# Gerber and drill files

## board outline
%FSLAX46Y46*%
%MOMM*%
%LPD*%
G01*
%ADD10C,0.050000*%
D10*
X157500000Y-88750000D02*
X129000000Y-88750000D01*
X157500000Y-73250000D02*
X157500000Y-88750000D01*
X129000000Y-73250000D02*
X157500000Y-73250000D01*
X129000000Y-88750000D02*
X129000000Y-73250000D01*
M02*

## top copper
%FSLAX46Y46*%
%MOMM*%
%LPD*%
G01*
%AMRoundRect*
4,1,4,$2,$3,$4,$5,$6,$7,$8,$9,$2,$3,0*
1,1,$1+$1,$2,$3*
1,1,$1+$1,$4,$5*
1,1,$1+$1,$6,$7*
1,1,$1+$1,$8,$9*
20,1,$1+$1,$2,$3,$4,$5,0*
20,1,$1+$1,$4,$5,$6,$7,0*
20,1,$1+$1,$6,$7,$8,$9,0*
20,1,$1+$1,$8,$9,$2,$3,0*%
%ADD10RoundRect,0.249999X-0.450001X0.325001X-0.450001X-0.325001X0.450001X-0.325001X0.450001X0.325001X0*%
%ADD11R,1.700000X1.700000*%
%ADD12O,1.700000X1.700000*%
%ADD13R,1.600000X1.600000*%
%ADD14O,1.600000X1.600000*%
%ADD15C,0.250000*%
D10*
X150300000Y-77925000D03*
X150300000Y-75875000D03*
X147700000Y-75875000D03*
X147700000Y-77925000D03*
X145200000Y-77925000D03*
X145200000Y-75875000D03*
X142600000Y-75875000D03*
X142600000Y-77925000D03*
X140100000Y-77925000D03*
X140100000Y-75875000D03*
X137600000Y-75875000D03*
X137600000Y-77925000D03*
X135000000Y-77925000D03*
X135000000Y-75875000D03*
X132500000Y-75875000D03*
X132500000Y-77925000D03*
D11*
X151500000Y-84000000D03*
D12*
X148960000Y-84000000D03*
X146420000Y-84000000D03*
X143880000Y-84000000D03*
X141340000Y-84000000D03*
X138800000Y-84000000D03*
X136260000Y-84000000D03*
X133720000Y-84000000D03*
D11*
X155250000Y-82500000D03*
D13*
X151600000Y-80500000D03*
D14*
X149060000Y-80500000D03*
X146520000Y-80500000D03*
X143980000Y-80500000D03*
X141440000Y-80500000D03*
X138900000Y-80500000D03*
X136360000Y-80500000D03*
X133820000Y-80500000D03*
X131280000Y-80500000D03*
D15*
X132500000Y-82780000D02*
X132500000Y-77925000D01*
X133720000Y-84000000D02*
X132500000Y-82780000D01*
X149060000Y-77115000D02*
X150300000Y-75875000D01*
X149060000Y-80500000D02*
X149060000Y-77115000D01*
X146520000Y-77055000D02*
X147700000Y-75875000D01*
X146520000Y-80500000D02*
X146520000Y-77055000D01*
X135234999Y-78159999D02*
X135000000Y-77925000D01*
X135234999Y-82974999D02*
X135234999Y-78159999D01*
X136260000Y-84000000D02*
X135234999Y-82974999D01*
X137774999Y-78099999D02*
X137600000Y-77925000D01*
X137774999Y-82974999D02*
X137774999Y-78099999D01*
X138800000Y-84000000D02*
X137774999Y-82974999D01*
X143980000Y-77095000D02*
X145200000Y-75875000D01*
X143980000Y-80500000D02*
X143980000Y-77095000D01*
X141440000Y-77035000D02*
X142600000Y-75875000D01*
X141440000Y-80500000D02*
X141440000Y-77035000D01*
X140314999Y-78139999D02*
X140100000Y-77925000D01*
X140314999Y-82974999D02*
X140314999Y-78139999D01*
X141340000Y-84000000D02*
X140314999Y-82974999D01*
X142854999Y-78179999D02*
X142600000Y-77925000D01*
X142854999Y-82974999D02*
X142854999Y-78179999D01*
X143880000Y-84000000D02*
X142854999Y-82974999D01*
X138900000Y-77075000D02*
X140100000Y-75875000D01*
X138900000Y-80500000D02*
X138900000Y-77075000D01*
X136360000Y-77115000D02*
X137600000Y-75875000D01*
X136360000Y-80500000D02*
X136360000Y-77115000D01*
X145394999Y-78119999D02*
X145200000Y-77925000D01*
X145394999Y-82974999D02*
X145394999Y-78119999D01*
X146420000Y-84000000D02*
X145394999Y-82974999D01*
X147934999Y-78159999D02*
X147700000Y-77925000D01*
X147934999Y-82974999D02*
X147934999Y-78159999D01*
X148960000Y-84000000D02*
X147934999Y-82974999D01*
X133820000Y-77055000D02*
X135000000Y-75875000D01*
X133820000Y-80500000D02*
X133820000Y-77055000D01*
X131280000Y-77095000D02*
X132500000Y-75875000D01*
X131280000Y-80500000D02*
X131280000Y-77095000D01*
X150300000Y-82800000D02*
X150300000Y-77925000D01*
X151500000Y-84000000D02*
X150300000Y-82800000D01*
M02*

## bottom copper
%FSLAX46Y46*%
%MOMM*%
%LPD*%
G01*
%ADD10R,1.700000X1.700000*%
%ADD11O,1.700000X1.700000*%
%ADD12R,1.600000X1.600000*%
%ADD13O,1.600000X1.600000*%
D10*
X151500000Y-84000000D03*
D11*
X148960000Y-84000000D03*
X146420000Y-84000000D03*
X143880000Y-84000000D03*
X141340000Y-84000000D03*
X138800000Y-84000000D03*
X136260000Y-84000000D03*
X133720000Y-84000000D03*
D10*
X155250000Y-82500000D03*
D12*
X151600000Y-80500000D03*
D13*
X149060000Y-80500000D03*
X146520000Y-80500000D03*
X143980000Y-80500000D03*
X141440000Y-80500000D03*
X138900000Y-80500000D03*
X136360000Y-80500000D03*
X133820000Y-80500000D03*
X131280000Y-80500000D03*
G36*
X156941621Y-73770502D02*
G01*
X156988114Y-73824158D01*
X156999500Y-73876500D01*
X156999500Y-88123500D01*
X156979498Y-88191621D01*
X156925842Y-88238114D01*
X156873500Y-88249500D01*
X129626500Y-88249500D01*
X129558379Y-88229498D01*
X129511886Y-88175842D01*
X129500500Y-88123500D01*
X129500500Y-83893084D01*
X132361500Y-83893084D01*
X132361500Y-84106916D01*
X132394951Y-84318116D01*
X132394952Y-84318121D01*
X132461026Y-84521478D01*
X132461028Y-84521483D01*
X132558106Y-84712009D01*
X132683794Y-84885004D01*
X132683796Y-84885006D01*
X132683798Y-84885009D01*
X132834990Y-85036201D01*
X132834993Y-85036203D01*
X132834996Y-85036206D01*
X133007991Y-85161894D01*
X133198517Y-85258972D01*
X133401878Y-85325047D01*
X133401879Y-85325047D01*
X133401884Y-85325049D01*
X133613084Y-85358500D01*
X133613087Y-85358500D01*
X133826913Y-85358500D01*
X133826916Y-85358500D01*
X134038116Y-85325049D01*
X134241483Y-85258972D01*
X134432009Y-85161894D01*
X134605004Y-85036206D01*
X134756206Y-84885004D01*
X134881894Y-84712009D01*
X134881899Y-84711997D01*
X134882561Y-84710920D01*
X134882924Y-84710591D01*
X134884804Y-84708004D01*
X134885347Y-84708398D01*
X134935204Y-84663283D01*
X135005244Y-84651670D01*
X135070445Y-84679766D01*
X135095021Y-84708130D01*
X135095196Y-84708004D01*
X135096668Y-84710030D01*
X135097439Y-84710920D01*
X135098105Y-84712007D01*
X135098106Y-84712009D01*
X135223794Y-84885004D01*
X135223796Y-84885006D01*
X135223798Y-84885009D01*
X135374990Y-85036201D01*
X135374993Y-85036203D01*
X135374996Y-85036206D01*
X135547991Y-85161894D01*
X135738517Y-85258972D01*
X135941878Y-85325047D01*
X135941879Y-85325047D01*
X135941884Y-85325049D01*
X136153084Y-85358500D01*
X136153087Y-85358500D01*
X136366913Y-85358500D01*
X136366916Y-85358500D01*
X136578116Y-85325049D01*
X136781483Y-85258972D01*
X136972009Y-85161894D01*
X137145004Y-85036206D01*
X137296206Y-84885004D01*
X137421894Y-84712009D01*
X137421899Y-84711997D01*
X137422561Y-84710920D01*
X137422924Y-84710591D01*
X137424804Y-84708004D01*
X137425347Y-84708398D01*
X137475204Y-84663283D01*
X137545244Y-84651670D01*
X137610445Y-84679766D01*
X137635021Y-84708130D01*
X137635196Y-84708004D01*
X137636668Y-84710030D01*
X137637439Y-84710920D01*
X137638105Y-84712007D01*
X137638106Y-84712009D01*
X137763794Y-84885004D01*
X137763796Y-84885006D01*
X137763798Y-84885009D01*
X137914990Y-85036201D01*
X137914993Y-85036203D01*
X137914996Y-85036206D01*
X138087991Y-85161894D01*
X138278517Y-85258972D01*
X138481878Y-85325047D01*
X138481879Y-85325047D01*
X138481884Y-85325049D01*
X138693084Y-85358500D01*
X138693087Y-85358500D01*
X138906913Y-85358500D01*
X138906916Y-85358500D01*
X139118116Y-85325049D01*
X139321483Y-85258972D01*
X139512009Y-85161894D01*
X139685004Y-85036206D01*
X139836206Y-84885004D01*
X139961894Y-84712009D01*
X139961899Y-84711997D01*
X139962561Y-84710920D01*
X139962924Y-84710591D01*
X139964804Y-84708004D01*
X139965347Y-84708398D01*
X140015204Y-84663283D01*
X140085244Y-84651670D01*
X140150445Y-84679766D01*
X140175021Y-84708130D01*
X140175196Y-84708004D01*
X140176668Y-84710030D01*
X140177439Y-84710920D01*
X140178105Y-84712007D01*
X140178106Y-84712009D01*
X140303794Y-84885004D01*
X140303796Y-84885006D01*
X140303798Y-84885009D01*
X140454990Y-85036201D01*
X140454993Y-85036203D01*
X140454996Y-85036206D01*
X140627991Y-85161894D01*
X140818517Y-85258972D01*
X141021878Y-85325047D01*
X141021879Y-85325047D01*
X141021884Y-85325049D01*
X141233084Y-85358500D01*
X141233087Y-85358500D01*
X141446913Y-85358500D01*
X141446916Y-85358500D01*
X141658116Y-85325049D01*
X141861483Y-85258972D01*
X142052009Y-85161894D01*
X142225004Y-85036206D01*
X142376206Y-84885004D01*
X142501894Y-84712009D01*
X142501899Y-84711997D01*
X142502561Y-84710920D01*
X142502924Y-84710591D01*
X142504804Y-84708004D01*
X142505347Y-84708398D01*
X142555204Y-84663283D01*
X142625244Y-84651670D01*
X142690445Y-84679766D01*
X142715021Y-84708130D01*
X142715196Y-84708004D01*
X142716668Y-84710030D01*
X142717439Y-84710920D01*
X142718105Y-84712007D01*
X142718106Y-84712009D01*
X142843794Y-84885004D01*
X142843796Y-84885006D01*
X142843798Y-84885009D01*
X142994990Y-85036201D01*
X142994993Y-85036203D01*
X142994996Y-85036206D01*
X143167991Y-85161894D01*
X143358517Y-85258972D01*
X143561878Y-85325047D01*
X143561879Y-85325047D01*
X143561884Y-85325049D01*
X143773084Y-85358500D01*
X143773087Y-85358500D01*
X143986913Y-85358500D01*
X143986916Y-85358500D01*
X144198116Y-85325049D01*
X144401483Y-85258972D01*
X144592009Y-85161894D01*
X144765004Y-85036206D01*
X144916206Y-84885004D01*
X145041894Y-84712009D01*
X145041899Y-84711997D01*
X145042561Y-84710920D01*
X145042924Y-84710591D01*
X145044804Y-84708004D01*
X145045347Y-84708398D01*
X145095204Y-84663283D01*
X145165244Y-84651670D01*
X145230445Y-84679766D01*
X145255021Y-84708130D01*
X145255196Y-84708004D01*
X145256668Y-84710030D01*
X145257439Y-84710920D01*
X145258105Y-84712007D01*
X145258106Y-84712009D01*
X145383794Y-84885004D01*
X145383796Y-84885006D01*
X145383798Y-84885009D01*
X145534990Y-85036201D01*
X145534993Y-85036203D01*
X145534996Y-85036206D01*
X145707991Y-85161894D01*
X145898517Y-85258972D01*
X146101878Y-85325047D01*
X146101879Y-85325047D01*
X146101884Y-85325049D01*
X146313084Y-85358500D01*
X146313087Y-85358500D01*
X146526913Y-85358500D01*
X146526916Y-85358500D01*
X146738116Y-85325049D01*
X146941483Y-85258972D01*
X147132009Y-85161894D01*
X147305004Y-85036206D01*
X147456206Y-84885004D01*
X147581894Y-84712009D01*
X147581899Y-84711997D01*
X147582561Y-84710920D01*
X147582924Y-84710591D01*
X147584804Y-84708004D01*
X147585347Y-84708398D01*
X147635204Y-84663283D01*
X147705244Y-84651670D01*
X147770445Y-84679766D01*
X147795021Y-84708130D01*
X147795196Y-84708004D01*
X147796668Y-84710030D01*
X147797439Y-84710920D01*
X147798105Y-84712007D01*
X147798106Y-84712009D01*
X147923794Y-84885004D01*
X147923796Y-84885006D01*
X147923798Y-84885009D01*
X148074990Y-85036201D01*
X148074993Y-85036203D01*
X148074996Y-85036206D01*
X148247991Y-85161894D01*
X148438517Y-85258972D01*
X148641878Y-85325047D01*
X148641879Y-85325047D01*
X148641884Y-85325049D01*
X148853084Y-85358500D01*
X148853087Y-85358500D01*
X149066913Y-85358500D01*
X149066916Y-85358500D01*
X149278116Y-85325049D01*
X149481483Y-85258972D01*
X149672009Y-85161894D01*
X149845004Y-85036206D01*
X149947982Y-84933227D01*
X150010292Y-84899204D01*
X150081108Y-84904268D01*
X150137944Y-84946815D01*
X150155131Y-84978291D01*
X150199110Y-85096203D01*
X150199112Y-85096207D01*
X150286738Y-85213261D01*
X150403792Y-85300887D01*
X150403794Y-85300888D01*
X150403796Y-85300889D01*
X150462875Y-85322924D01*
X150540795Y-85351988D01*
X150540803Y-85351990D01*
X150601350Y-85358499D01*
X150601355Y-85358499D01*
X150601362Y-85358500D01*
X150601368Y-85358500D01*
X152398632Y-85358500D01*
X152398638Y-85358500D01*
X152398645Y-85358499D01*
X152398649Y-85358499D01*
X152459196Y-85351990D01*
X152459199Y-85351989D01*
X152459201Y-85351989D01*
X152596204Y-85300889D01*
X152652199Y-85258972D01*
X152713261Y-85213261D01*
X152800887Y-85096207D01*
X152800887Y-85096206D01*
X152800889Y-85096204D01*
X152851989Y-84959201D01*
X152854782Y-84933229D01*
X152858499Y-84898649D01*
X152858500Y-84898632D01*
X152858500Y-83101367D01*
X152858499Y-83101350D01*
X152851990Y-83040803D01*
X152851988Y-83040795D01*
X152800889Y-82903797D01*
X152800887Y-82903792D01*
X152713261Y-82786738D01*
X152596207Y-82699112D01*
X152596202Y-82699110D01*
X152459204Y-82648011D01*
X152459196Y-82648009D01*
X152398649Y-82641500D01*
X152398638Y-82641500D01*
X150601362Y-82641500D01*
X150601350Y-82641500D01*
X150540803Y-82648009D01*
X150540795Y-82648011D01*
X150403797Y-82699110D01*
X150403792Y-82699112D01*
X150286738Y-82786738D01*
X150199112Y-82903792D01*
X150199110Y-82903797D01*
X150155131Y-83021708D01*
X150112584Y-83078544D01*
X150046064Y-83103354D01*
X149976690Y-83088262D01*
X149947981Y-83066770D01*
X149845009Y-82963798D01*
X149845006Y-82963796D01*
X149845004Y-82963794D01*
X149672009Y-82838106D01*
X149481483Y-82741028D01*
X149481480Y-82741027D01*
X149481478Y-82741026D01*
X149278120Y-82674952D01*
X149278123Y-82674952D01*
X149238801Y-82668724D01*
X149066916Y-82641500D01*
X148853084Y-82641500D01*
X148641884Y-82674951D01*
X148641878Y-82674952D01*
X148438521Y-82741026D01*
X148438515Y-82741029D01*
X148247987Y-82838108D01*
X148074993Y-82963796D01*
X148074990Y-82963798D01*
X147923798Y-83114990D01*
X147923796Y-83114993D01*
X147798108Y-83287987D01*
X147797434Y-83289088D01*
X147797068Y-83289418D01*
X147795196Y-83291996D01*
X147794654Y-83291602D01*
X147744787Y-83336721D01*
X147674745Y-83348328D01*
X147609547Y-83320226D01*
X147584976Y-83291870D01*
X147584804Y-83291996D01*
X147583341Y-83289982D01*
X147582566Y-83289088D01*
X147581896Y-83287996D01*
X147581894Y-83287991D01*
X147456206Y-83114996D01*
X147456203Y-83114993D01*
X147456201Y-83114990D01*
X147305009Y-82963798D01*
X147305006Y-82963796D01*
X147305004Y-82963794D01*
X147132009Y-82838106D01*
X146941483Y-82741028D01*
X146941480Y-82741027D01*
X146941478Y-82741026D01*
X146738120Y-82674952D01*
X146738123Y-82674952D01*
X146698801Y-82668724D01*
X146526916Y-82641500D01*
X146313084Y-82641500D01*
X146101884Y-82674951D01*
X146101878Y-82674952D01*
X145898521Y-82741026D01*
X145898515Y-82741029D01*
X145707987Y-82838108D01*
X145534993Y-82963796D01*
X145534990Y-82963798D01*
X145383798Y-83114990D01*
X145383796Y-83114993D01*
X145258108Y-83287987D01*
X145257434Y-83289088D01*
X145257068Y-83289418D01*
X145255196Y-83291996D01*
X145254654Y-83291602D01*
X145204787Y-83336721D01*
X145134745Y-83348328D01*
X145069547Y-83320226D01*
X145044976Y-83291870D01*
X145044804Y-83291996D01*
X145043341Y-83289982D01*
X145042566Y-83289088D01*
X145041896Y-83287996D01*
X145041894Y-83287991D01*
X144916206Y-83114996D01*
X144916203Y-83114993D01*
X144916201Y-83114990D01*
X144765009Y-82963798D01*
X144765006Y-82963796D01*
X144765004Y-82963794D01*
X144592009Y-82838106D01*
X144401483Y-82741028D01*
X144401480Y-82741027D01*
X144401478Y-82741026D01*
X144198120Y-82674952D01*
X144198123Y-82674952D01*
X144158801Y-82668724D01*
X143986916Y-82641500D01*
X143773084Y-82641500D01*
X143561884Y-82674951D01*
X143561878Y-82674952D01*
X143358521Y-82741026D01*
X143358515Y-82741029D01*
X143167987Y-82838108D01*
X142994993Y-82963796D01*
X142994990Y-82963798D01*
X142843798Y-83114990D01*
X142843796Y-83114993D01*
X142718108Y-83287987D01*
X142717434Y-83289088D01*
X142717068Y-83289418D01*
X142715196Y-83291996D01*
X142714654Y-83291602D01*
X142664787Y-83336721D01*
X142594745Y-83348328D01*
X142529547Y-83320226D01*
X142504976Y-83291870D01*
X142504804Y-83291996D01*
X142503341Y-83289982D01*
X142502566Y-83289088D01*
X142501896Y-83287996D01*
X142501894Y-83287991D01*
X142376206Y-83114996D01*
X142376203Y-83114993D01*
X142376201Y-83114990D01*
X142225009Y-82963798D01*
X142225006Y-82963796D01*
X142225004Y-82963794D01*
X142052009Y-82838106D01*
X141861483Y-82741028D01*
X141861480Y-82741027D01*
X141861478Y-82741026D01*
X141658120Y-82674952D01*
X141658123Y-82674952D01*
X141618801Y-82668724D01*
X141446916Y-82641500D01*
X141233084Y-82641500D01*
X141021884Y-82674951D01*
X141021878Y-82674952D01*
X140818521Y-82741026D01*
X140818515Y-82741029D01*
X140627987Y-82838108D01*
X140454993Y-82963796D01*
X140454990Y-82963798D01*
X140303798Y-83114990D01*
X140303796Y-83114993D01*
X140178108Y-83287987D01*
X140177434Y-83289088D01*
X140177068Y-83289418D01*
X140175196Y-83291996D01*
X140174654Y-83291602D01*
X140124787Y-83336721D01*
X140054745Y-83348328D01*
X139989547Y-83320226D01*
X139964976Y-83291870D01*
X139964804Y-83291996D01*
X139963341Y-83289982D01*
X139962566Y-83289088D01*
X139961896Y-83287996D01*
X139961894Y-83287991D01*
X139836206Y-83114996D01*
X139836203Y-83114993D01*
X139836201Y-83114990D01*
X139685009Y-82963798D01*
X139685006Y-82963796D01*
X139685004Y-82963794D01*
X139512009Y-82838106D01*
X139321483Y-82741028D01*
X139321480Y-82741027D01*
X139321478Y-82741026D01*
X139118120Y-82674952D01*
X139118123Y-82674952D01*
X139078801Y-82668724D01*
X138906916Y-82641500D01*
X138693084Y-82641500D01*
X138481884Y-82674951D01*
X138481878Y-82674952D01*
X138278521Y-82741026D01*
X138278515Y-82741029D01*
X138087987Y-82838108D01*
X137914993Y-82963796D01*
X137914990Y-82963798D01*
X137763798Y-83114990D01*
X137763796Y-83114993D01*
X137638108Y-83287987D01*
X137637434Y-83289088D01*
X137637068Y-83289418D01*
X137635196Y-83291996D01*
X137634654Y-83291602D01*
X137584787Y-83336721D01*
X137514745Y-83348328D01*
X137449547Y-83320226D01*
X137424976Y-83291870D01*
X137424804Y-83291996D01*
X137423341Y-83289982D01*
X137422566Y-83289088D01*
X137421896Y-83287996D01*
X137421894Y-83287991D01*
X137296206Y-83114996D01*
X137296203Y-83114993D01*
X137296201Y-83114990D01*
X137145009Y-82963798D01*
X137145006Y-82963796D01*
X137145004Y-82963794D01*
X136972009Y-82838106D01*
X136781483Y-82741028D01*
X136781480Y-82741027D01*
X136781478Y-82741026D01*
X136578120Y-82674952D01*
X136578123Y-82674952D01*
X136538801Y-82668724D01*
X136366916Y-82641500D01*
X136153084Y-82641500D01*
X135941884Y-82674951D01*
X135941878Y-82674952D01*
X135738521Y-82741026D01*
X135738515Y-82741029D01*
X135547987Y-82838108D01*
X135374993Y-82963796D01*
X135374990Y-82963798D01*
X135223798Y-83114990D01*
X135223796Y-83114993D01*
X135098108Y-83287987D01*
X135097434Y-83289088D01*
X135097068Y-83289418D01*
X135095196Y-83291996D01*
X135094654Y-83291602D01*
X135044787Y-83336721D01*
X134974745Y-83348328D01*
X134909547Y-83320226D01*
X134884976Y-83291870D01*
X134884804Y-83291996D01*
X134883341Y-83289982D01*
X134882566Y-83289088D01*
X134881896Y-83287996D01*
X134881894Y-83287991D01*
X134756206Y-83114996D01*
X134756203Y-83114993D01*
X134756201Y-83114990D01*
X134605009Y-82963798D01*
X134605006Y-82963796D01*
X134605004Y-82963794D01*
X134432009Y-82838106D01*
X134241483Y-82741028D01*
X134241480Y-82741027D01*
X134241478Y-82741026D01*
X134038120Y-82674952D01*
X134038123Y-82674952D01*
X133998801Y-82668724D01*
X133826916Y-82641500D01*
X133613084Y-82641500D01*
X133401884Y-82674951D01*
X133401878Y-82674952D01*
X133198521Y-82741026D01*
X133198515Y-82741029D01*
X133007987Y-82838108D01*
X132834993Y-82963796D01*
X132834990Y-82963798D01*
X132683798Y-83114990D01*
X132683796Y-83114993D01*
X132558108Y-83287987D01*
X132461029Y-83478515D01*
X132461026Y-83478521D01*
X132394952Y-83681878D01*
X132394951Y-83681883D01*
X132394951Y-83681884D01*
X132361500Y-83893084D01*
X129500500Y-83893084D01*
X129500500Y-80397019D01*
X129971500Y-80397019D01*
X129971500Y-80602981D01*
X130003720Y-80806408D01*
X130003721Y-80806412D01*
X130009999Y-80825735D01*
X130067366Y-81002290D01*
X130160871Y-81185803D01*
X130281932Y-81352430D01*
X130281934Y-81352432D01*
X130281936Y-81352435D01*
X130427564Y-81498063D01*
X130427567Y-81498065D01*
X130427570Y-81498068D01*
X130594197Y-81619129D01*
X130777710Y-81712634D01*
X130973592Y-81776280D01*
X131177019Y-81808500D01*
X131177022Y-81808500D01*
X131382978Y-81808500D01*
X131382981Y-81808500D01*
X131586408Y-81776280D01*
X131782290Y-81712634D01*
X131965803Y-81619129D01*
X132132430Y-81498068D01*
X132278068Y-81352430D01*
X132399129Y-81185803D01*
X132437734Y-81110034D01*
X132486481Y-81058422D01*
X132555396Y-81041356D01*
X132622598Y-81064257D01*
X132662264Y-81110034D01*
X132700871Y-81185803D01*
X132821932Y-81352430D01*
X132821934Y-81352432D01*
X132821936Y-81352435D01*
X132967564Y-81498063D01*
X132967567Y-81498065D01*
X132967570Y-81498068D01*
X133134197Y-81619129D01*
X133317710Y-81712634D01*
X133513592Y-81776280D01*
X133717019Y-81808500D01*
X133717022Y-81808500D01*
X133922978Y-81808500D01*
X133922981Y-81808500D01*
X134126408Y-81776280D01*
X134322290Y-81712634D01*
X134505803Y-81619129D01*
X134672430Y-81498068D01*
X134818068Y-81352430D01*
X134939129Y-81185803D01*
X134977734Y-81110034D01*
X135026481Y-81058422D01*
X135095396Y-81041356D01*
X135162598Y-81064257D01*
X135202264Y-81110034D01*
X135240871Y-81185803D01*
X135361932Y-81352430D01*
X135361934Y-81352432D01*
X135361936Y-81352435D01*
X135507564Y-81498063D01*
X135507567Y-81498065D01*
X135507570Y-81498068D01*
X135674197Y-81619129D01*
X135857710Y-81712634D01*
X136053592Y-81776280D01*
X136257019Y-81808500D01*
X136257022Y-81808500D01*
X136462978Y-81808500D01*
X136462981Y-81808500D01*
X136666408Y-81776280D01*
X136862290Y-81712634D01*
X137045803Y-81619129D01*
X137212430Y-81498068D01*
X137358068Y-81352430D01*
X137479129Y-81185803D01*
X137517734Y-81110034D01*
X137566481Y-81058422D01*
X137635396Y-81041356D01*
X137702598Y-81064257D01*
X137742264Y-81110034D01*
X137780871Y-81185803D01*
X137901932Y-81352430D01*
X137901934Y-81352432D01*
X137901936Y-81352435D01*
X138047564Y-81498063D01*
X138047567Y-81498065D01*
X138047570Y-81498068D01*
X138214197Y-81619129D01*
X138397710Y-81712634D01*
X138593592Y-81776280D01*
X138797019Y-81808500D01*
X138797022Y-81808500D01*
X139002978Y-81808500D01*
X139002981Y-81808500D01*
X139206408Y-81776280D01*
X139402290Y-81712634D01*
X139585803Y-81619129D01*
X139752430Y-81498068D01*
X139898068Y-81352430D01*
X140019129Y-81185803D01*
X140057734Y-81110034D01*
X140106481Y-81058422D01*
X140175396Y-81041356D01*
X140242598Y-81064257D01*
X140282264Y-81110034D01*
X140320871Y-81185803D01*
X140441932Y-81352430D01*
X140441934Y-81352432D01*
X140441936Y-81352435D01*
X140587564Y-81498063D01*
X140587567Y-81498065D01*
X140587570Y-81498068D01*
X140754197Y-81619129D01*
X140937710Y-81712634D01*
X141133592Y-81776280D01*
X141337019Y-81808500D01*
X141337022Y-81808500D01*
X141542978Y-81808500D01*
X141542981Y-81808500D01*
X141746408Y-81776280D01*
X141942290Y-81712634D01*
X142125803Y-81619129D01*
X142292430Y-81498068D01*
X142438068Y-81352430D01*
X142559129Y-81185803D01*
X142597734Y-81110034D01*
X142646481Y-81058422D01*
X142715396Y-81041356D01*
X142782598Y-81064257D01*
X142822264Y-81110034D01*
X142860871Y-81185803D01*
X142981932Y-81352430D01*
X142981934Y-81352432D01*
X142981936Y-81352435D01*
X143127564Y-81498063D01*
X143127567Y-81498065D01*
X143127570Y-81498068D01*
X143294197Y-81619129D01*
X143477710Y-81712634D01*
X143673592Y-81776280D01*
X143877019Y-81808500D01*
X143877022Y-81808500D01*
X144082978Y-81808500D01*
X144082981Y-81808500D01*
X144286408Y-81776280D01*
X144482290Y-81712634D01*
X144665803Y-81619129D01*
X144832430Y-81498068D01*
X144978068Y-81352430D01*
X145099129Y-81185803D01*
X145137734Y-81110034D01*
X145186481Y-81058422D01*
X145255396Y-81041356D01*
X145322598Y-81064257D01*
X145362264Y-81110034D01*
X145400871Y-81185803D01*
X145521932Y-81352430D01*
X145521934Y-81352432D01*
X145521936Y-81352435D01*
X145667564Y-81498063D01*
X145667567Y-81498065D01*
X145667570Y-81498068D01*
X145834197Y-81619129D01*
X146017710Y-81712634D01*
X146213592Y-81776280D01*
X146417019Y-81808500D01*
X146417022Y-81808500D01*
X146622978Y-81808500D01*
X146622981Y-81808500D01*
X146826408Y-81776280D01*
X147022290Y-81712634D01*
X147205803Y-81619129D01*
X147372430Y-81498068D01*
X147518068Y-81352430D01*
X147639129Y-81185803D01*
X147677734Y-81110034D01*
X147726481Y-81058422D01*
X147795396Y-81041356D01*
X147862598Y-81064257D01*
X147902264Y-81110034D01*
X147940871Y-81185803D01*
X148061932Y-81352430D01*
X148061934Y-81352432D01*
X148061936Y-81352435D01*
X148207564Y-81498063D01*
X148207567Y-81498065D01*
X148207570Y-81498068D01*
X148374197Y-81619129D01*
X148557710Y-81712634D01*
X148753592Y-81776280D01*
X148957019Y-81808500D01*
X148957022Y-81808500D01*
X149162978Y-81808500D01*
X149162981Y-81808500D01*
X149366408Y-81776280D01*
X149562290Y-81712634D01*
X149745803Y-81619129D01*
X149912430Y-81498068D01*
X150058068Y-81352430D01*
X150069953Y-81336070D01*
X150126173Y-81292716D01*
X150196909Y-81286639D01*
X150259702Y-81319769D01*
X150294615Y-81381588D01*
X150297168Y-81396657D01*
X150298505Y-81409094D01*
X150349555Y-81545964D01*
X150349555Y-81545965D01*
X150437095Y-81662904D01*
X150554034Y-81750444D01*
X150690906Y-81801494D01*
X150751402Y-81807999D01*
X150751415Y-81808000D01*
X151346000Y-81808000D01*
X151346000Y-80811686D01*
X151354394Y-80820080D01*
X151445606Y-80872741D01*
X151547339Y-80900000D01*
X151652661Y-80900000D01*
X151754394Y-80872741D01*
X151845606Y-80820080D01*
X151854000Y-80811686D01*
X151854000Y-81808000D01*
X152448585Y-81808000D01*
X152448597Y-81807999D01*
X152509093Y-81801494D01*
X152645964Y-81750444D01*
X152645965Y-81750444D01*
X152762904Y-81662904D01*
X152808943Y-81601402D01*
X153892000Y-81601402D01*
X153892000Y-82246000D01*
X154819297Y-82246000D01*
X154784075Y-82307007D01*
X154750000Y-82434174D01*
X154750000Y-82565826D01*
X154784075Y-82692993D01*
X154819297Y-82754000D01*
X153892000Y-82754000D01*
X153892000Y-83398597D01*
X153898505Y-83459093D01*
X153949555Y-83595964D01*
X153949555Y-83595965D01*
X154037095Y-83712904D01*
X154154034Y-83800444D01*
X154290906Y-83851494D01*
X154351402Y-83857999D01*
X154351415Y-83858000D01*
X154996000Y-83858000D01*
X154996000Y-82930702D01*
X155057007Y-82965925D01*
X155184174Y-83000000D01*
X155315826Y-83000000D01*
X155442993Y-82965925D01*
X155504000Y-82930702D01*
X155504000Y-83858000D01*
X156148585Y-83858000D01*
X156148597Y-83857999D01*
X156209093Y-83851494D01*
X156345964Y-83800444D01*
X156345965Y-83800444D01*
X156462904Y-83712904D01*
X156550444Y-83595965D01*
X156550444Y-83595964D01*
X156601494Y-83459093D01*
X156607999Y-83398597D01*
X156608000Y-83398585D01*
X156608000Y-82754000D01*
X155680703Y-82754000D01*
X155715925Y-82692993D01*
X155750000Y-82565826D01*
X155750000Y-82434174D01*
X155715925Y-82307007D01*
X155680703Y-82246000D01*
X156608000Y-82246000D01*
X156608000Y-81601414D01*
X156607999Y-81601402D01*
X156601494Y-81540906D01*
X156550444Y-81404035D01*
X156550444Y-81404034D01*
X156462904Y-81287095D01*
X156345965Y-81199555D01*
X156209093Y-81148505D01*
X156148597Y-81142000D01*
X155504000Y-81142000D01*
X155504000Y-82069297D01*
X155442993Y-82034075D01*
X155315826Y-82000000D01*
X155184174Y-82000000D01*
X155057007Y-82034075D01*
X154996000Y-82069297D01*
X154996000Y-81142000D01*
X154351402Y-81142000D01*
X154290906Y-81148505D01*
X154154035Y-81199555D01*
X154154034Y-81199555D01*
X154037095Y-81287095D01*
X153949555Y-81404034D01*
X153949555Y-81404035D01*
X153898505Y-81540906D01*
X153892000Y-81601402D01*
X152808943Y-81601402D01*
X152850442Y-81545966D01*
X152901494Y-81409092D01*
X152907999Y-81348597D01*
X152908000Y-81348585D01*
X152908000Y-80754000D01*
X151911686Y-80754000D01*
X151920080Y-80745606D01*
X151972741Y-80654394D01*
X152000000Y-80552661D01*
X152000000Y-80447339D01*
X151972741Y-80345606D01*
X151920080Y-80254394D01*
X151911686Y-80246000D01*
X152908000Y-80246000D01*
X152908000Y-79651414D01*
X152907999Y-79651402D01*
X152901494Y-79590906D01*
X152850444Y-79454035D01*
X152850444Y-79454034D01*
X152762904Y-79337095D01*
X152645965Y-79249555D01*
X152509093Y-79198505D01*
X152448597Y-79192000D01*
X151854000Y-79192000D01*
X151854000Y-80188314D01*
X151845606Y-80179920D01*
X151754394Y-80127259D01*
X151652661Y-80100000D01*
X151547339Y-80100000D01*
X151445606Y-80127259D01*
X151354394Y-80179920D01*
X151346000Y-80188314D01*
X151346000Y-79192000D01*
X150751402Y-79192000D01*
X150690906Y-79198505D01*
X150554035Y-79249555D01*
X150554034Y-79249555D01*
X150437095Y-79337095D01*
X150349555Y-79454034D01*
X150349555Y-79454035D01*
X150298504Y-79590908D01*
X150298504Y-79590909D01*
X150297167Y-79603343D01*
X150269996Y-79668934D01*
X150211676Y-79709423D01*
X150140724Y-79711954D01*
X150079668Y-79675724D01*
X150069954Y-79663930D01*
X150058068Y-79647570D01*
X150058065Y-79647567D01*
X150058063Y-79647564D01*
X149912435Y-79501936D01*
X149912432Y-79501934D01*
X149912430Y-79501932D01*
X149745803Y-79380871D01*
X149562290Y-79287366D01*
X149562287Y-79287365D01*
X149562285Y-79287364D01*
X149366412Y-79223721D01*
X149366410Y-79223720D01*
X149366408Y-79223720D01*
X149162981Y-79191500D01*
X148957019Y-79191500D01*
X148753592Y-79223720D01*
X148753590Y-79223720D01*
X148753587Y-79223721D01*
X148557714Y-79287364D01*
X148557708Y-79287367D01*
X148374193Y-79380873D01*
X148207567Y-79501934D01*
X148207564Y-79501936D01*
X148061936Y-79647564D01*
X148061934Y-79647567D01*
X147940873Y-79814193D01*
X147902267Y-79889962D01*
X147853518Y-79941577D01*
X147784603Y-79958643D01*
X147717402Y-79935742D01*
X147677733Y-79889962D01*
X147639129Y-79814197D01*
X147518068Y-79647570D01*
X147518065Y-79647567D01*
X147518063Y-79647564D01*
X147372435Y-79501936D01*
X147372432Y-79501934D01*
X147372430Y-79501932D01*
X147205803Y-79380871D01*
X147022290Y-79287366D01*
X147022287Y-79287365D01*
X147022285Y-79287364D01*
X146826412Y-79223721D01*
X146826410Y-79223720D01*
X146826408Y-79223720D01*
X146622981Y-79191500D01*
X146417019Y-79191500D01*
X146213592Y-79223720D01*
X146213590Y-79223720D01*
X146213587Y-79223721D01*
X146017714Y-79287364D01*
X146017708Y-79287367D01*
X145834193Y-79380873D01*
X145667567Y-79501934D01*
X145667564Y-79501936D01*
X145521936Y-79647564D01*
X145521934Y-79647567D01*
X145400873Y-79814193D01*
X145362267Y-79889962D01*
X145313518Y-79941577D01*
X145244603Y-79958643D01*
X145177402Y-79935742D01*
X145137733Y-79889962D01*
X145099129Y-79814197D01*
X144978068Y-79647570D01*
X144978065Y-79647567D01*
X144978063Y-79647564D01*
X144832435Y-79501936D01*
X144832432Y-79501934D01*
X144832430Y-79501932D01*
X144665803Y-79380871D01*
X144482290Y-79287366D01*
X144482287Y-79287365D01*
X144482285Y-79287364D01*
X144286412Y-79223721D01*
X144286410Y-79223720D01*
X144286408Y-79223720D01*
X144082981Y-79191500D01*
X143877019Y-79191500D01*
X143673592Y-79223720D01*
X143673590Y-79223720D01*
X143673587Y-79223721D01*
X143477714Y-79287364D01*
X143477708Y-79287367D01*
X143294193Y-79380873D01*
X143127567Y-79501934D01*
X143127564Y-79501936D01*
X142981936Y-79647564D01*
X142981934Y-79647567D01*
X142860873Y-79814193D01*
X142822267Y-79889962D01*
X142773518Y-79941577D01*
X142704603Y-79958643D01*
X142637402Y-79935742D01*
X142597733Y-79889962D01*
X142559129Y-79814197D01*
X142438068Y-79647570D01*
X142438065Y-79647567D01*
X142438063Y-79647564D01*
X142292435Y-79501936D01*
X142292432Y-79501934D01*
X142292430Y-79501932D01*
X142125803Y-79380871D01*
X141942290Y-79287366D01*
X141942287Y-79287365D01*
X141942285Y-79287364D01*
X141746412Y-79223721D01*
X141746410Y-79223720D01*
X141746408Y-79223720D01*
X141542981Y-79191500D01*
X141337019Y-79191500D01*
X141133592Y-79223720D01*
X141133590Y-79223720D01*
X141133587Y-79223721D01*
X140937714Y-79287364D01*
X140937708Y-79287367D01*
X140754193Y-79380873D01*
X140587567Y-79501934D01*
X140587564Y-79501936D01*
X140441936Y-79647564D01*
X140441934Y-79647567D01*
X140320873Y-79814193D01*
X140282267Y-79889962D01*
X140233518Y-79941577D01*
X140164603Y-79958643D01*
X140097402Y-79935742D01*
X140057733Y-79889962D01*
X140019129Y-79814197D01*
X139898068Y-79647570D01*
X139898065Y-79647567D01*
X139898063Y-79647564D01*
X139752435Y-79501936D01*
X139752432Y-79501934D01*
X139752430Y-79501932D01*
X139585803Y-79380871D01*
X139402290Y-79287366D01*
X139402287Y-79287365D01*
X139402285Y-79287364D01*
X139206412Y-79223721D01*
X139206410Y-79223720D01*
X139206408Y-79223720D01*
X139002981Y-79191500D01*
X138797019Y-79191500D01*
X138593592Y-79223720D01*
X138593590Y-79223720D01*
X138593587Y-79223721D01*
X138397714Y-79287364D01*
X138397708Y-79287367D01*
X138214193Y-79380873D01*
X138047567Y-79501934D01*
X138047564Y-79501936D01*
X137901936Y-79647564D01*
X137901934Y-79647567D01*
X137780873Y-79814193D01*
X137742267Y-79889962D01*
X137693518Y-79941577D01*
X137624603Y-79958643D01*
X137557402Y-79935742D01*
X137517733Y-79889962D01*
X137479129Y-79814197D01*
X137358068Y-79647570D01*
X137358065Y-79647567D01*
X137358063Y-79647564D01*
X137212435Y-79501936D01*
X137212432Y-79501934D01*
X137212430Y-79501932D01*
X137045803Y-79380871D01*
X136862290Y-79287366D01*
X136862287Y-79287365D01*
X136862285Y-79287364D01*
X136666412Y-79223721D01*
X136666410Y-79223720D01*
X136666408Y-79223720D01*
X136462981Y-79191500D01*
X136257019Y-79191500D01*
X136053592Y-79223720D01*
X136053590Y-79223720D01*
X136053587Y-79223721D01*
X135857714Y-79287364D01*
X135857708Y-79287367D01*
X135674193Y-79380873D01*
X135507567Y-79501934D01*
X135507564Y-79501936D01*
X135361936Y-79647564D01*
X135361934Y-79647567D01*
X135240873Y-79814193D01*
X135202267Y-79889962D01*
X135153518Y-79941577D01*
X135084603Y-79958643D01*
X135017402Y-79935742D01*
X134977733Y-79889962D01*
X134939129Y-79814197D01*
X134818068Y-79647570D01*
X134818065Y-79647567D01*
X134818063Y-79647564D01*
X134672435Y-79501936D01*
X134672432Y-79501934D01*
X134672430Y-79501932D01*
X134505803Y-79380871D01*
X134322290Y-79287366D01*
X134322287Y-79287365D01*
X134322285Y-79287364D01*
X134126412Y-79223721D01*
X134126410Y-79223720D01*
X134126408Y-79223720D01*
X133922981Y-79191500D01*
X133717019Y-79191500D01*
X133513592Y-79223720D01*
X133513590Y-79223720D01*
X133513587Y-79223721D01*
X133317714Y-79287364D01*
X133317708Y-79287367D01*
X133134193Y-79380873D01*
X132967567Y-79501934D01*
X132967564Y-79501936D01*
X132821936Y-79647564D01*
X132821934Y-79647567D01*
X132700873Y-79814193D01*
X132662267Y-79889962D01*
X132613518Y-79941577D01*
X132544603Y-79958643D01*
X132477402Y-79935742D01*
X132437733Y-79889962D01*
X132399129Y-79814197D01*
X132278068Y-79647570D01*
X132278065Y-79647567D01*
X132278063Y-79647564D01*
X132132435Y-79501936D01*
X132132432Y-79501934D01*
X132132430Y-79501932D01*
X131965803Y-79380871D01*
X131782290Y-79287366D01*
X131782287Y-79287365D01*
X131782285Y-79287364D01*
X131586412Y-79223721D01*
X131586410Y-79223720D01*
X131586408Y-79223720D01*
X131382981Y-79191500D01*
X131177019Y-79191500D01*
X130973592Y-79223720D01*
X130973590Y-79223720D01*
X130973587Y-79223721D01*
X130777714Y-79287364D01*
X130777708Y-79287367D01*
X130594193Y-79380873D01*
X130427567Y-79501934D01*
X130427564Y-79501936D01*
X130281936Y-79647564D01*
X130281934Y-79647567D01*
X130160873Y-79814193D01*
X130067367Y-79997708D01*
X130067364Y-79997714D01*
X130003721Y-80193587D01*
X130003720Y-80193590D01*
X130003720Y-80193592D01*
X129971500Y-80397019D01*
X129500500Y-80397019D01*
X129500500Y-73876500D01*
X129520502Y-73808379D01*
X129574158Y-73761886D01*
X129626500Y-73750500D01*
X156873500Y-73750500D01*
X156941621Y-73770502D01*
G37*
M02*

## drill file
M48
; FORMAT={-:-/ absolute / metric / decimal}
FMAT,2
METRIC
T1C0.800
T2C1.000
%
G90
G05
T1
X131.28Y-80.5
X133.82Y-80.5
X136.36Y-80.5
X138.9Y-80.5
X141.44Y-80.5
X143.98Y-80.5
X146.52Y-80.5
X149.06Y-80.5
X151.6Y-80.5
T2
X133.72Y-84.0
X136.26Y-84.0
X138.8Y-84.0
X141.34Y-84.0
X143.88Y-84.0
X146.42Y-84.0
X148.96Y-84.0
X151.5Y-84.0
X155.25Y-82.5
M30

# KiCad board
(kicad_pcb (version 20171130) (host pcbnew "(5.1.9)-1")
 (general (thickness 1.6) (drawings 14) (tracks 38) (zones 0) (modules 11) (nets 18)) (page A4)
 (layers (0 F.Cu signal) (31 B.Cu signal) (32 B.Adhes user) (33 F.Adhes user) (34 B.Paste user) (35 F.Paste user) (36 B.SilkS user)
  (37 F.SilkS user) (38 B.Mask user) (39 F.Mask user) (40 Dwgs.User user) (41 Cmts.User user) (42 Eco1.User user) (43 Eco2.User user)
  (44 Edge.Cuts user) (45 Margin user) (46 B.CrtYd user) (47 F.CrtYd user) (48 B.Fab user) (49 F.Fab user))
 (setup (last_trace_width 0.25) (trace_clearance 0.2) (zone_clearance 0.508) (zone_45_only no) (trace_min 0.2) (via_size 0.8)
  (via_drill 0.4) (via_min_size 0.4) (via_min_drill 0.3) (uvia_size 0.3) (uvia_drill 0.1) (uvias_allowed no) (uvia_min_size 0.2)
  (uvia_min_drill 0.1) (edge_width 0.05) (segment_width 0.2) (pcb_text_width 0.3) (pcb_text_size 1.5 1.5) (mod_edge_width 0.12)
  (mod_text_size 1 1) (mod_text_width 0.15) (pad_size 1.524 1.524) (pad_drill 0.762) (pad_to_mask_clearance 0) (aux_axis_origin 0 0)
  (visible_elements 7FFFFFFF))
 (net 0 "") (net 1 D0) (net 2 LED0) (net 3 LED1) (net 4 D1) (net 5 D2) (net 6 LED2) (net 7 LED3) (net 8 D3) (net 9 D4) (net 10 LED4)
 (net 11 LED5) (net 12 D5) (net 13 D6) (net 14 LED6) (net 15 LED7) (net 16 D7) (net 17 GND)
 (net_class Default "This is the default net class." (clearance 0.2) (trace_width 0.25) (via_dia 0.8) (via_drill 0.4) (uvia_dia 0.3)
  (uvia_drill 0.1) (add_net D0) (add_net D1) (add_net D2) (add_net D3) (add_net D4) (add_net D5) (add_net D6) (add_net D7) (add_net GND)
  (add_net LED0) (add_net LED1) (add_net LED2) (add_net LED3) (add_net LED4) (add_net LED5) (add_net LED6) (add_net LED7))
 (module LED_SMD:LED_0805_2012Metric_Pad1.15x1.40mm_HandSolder (layer F.Cu) (at 150.3 76.9 270)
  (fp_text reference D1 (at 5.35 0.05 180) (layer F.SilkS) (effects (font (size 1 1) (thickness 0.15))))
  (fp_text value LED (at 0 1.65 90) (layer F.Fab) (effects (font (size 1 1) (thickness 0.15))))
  (pad 2 smd roundrect (at 1.025 0 270) (size 1.15 1.4) (layers F.Cu F.Paste F.Mask) (roundrect_rratio 0.2173904347826087) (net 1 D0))
  (pad 1 smd roundrect (at -1.025 0 270) (size 1.15 1.4) (layers F.Cu F.Paste F.Mask) (roundrect_rratio 0.2173904347826087) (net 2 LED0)))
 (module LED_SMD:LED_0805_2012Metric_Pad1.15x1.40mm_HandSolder (layer F.Cu) (at 147.7 76.9 270)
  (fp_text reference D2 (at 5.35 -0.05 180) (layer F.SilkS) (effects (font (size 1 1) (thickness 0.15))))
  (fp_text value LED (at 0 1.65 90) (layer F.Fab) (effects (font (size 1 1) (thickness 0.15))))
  (pad 1 smd roundrect (at -1.025 0 270) (size 1.15 1.4) (layers F.Cu F.Paste F.Mask) (roundrect_rratio 0.2173904347826087) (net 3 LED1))
  (pad 2 smd roundrect (at 1.025 0 270) (size 1.15 1.4) (layers F.Cu F.Paste F.Mask) (roundrect_rratio 0.2173904347826087) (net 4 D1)))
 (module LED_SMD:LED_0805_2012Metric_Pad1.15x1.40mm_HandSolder (layer F.Cu) (at 145.2 76.9 270)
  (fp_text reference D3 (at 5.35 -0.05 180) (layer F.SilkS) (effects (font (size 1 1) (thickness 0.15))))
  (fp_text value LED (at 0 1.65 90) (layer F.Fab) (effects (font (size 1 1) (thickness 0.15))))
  (pad 2 smd roundrect (at 1.025 0 270) (size 1.15 1.4) (layers F.Cu F.Paste F.Mask) (roundrect_rratio 0.2173904347826087) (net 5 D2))
  (pad 1 smd roundrect (at -1.025 0 270) (size 1.15 1.4) (layers F.Cu F.Paste F.Mask) (roundrect_rratio 0.2173904347826087) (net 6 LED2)))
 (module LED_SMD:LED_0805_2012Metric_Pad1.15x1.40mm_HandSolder (layer F.Cu) (at 142.6 76.9 270)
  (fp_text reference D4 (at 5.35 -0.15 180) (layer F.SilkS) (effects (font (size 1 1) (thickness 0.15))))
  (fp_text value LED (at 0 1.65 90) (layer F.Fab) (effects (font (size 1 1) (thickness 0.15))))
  (pad 1 smd roundrect (at -1.025 0 270) (size 1.15 1.4) (layers F.Cu F.Paste F.Mask) (roundrect_rratio 0.2173904347826087) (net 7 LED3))
  (pad 2 smd roundrect (at 1.025 0 270) (size 1.15 1.4) (layers F.Cu F.Paste F.Mask) (roundrect_rratio 0.2173904347826087) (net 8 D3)))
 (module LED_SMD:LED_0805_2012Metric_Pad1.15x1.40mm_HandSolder (layer F.Cu) (at 140.1 76.9 270)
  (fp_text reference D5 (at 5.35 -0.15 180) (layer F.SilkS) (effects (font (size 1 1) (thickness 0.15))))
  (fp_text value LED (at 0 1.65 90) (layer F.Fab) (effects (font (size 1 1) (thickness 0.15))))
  (pad 2 smd roundrect (at 1.025 0 270) (size 1.15 1.4) (layers F.Cu F.Paste F.Mask) (roundrect_rratio 0.2173904347826087) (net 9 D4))
  (pad 1 smd roundrect (at -1.025 0 270) (size 1.15 1.4) (layers F.Cu F.Paste F.Mask) (roundrect_rratio 0.2173904347826087) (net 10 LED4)))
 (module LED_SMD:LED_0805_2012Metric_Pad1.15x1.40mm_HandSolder (layer F.Cu) (at 137.6 76.9 270)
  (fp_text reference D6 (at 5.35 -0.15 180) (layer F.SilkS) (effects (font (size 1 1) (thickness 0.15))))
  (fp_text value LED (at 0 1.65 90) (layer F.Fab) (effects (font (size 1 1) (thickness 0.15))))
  (pad 1 smd roundrect (at -1.025 0 270) (size 1.15 1.4) (layers F.Cu F.Paste F.Mask) (roundrect_rratio 0.2173904347826087) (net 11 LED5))
  (pad 2 smd roundrect (at 1.025 0 270) (size 1.15 1.4) (layers F.Cu F.Paste F.Mask) (roundrect_rratio 0.2173904347826087) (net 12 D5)))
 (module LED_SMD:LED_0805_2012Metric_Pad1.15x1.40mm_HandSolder (layer F.Cu) (at 135 76.9 270)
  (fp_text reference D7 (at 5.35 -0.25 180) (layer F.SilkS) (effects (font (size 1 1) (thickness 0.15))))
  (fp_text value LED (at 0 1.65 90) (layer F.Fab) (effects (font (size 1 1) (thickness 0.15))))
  (pad 2 smd roundrect (at 1.025 0 270) (size 1.15 1.4) (layers F.Cu F.Paste F.Mask) (roundrect_rratio 0.2173904347826087) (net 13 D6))
  (pad 1 smd roundrect (at -1.025 0 270) (size 1.15 1.4) (layers F.Cu F.Paste F.Mask) (roundrect_rratio 0.2173904347826087) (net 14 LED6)))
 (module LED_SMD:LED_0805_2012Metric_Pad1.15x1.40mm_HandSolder (layer F.Cu) (at 132.5 76.9 270)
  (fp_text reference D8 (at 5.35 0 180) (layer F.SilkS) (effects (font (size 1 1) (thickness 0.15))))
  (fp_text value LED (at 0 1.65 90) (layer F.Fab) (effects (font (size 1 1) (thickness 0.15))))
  (pad 1 smd roundrect (at -1.025 0 270) (size 1.15 1.4) (layers F.Cu F.Paste F.Mask) (roundrect_rratio 0.2173904347826087) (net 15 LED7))
  (pad 2 smd roundrect (at 1.025 0 270) (size 1.15 1.4) (layers F.Cu F.Paste F.Mask) (roundrect_rratio 0.2173904347826087) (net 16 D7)))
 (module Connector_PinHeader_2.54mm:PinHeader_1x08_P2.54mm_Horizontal (layer F.Cu) (at 151.5 84 270)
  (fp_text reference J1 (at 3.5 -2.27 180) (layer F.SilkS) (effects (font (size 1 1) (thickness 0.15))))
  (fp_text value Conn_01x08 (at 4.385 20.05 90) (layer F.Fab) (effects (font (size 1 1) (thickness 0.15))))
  (pad 1 thru_hole rect (at 0 0 270) (size 1.7 1.7) (drill 1) (layers *.Cu *.Mask) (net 1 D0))
  (pad 2 thru_hole oval (at 0 2.54 270) (size 1.7 1.7) (drill 1) (layers *.Cu *.Mask) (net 4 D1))
  (pad 3 thru_hole oval (at 0 5.08 270) (size 1.7 1.7) (drill 1) (layers *.Cu *.Mask) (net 5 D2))
  (pad 4 thru_hole oval (at 0 7.62 270) (size 1.7 1.7) (drill 1) (layers *.Cu *.Mask) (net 8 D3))
  (pad 5 thru_hole oval (at 0 10.16 270) (size 1.7 1.7) (drill 1) (layers *.Cu *.Mask) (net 9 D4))
  (pad 6 thru_hole oval (at 0 12.7 270) (size 1.7 1.7) (drill 1) (layers *.Cu *.Mask) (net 12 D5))
  (pad 7 thru_hole oval (at 0 15.24 270) (size 1.7 1.7) (drill 1) (layers *.Cu *.Mask) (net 13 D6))
  (pad 8 thru_hole oval (at 0 17.78 270) (size 1.7 1.7) (drill 1) (layers *.Cu *.Mask) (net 16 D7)))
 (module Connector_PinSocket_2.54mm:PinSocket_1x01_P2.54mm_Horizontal (layer F.Cu) (at 155.25 82.5 270)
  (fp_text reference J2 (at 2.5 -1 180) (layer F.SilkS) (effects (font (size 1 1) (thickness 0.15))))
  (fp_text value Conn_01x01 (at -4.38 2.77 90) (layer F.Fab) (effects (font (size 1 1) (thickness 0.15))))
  (pad 1 thru_hole rect (at 0 0 270) (size 1.7 1.7) (drill 1) (layers *.Cu *.Mask) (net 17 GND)))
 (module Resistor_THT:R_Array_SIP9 (layer F.Cu) (at 151.6 80.5 180)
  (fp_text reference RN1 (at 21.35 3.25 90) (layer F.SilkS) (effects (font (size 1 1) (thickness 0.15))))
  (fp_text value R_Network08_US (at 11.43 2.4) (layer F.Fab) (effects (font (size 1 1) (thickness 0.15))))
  (pad 1 thru_hole rect (at 0 0 180) (size 1.6 1.6) (drill 0.8) (layers *.Cu *.Mask) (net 17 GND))
  (pad 2 thru_hole oval (at 2.54 0 180) (size 1.6 1.6) (drill 0.8) (layers *.Cu *.Mask) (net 2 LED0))
  (pad 3 thru_hole oval (at 5.08 0 180) (size 1.6 1.6) (drill 0.8) (layers *.Cu *.Mask) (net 3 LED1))
  (pad 4 thru_hole oval (at 7.62 0 180) (size 1.6 1.6) (drill 0.8) (layers *.Cu *.Mask) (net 6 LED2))
  (pad 5 thru_hole oval (at 10.16 0 180) (size 1.6 1.6) (drill 0.8) (layers *.Cu *.Mask) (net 7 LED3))
  (pad 6 thru_hole oval (at 12.7 0 180) (size 1.6 1.6) (drill 0.8) (layers *.Cu *.Mask) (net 10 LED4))
  (pad 7 thru_hole oval (at 15.24 0 180) (size 1.6 1.6) (drill 0.8) (layers *.Cu *.Mask) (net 11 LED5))
  (pad 8 thru_hole oval (at 17.78 0 180) (size 1.6 1.6) (drill 0.8) (layers *.Cu *.Mask) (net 14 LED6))
  (pad 9 thru_hole oval (at 20.32 0 180) (size 1.6 1.6) (drill 0.8) (layers *.Cu *.Mask) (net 15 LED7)))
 (gr_line (start 157.5 88.75) (end 129 88.75) (layer Edge.Cuts) (width 0.05))
 (gr_line (start 157.5 73.25) (end 157.5 88.75) (layer Edge.Cuts) (width 0.05))
 (gr_line (start 129 73.25) (end 157.5 73.25) (layer Edge.Cuts) (width 0.05))
 (gr_line (start 129 88.75) (end 129 73.25) (layer Edge.Cuts) (width 0.05))
 (segment (start 132.5 82.78) (end 132.5 77.925) (width 0.25) (layer F.Cu) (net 16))
 (segment (start 133.72 84) (end 132.5 82.78) (width 0.25) (layer F.Cu) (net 16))
 (segment (start 149.06 77.115) (end 150.3 75.875) (width 0.25) (layer F.Cu) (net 2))
 (segment (start 149.06 80.5) (end 149.06 77.115) (width 0.25) (layer F.Cu) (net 2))
 (segment (start 146.52 77.055) (end 147.7 75.875) (width 0.25) (layer F.Cu) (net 3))
 (segment (start 146.52 80.5) (end 146.52 77.055) (width 0.25) (layer F.Cu) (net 3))
 (segment (start 135.234999 78.159999) (end 135 77.925) (width 0.25) (layer F.Cu) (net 13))
 (segment (start 135.234999 82.974999) (end 135.234999 78.159999) (width 0.25) (layer F.Cu) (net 13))
 (segment (start 136.26 84) (end 135.234999 82.974999) (width 0.25) (layer F.Cu) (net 13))
 (segment (start 137.774999 78.099999) (end 137.6 77.925) (width 0.25) (layer F.Cu) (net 12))
 (segment (start 137.774999 82.974999) (end 137.774999 78.099999) (width 0.25) (layer F.Cu) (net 12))
 (segment (start 138.8 84) (end 137.774999 82.974999) (width 0.25) (layer F.Cu) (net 12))
 (segment (start 143.98 77.095) (end 145.2 75.875) (width 0.25) (layer F.Cu) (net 6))
 (segment (start 143.98 80.5) (end 143.98 77.095) (width 0.25) (layer F.Cu) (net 6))
 (segment (start 141.44 77.035) (end 142.6 75.875) (width 0.25) (layer F.Cu) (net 7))
 (segment (start 141.44 80.5) (end 141.44 77.035) (width 0.25) (layer F.Cu) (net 7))
 (segment (start 140.314999 78.139999) (end 140.1 77.925) (width 0.25) (layer F.Cu) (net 9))
 (segment (start 140.314999 82.974999) (end 140.314999 78.139999) (width 0.25) (layer F.Cu) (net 9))
 (segment (start 141.34 84) (end 140.314999 82.974999) (width 0.25) (layer F.Cu) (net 9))
 (segment (start 142.854999 78.179999) (end 142.6 77.925) (width 0.25) (layer F.Cu) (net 8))
 (segment (start 142.854999 82.974999) (end 142.854999 78.179999) (width 0.25) (layer F.Cu) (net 8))
 (segment (start 143.88 84) (end 142.854999 82.974999) (width 0.25) (layer F.Cu) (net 8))
 (segment (start 138.9 77.075) (end 140.1 75.875) (width 0.25) (layer F.Cu) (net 10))
 (segment (start 138.9 80.5) (end 138.9 77.075) (width 0.25) (layer F.Cu) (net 10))
 (segment (start 136.36 77.115) (end 137.6 75.875) (width 0.25) (layer F.Cu) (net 11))
 (segment (start 136.36 80.5) (end 136.36 77.115) (width 0.25) (layer F.Cu) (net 11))
 (segment (start 145.394999 78.119999) (end 145.2 77.925) (width 0.25) (layer F.Cu) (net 5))
 (segment (start 145.394999 82.974999) (end 145.394999 78.119999) (width 0.25) (layer F.Cu) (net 5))
 (segment (start 146.42 84) (end 145.394999 82.974999) (width 0.25) (layer F.Cu) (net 5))
 (segment (start 147.934999 78.159999) (end 147.7 77.925) (width 0.25) (layer F.Cu) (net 4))
 (segment (start 147.934999 82.974999) (end 147.934999 78.159999) (width 0.25) (layer F.Cu) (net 4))
 (segment (start 148.96 84) (end 147.934999 82.974999) (width 0.25) (layer F.Cu) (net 4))
 (segment (start 133.82 77.055) (end 135 75.875) (width 0.25) (layer F.Cu) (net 14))
 (segment (start 133.82 80.5) (end 133.82 77.055) (width 0.25) (layer F.Cu) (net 14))
 (segment (start 131.28 77.095) (end 132.5 75.875) (width 0.25) (layer F.Cu) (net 15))
 (segment (start 131.28 80.5) (end 131.28 77.095) (width 0.25) (layer F.Cu) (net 15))
 (segment (start 150.3 82.8) (end 150.3 77.925) (width 0.25) (layer F.Cu) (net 1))
 (segment (start 151.5 84) (end 150.3 82.8) (width 0.25) (layer F.Cu) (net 1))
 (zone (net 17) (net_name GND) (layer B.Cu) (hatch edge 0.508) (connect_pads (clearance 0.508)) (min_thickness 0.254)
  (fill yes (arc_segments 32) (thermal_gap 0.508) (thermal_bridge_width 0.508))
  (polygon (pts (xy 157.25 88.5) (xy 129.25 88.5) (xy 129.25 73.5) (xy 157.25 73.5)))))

